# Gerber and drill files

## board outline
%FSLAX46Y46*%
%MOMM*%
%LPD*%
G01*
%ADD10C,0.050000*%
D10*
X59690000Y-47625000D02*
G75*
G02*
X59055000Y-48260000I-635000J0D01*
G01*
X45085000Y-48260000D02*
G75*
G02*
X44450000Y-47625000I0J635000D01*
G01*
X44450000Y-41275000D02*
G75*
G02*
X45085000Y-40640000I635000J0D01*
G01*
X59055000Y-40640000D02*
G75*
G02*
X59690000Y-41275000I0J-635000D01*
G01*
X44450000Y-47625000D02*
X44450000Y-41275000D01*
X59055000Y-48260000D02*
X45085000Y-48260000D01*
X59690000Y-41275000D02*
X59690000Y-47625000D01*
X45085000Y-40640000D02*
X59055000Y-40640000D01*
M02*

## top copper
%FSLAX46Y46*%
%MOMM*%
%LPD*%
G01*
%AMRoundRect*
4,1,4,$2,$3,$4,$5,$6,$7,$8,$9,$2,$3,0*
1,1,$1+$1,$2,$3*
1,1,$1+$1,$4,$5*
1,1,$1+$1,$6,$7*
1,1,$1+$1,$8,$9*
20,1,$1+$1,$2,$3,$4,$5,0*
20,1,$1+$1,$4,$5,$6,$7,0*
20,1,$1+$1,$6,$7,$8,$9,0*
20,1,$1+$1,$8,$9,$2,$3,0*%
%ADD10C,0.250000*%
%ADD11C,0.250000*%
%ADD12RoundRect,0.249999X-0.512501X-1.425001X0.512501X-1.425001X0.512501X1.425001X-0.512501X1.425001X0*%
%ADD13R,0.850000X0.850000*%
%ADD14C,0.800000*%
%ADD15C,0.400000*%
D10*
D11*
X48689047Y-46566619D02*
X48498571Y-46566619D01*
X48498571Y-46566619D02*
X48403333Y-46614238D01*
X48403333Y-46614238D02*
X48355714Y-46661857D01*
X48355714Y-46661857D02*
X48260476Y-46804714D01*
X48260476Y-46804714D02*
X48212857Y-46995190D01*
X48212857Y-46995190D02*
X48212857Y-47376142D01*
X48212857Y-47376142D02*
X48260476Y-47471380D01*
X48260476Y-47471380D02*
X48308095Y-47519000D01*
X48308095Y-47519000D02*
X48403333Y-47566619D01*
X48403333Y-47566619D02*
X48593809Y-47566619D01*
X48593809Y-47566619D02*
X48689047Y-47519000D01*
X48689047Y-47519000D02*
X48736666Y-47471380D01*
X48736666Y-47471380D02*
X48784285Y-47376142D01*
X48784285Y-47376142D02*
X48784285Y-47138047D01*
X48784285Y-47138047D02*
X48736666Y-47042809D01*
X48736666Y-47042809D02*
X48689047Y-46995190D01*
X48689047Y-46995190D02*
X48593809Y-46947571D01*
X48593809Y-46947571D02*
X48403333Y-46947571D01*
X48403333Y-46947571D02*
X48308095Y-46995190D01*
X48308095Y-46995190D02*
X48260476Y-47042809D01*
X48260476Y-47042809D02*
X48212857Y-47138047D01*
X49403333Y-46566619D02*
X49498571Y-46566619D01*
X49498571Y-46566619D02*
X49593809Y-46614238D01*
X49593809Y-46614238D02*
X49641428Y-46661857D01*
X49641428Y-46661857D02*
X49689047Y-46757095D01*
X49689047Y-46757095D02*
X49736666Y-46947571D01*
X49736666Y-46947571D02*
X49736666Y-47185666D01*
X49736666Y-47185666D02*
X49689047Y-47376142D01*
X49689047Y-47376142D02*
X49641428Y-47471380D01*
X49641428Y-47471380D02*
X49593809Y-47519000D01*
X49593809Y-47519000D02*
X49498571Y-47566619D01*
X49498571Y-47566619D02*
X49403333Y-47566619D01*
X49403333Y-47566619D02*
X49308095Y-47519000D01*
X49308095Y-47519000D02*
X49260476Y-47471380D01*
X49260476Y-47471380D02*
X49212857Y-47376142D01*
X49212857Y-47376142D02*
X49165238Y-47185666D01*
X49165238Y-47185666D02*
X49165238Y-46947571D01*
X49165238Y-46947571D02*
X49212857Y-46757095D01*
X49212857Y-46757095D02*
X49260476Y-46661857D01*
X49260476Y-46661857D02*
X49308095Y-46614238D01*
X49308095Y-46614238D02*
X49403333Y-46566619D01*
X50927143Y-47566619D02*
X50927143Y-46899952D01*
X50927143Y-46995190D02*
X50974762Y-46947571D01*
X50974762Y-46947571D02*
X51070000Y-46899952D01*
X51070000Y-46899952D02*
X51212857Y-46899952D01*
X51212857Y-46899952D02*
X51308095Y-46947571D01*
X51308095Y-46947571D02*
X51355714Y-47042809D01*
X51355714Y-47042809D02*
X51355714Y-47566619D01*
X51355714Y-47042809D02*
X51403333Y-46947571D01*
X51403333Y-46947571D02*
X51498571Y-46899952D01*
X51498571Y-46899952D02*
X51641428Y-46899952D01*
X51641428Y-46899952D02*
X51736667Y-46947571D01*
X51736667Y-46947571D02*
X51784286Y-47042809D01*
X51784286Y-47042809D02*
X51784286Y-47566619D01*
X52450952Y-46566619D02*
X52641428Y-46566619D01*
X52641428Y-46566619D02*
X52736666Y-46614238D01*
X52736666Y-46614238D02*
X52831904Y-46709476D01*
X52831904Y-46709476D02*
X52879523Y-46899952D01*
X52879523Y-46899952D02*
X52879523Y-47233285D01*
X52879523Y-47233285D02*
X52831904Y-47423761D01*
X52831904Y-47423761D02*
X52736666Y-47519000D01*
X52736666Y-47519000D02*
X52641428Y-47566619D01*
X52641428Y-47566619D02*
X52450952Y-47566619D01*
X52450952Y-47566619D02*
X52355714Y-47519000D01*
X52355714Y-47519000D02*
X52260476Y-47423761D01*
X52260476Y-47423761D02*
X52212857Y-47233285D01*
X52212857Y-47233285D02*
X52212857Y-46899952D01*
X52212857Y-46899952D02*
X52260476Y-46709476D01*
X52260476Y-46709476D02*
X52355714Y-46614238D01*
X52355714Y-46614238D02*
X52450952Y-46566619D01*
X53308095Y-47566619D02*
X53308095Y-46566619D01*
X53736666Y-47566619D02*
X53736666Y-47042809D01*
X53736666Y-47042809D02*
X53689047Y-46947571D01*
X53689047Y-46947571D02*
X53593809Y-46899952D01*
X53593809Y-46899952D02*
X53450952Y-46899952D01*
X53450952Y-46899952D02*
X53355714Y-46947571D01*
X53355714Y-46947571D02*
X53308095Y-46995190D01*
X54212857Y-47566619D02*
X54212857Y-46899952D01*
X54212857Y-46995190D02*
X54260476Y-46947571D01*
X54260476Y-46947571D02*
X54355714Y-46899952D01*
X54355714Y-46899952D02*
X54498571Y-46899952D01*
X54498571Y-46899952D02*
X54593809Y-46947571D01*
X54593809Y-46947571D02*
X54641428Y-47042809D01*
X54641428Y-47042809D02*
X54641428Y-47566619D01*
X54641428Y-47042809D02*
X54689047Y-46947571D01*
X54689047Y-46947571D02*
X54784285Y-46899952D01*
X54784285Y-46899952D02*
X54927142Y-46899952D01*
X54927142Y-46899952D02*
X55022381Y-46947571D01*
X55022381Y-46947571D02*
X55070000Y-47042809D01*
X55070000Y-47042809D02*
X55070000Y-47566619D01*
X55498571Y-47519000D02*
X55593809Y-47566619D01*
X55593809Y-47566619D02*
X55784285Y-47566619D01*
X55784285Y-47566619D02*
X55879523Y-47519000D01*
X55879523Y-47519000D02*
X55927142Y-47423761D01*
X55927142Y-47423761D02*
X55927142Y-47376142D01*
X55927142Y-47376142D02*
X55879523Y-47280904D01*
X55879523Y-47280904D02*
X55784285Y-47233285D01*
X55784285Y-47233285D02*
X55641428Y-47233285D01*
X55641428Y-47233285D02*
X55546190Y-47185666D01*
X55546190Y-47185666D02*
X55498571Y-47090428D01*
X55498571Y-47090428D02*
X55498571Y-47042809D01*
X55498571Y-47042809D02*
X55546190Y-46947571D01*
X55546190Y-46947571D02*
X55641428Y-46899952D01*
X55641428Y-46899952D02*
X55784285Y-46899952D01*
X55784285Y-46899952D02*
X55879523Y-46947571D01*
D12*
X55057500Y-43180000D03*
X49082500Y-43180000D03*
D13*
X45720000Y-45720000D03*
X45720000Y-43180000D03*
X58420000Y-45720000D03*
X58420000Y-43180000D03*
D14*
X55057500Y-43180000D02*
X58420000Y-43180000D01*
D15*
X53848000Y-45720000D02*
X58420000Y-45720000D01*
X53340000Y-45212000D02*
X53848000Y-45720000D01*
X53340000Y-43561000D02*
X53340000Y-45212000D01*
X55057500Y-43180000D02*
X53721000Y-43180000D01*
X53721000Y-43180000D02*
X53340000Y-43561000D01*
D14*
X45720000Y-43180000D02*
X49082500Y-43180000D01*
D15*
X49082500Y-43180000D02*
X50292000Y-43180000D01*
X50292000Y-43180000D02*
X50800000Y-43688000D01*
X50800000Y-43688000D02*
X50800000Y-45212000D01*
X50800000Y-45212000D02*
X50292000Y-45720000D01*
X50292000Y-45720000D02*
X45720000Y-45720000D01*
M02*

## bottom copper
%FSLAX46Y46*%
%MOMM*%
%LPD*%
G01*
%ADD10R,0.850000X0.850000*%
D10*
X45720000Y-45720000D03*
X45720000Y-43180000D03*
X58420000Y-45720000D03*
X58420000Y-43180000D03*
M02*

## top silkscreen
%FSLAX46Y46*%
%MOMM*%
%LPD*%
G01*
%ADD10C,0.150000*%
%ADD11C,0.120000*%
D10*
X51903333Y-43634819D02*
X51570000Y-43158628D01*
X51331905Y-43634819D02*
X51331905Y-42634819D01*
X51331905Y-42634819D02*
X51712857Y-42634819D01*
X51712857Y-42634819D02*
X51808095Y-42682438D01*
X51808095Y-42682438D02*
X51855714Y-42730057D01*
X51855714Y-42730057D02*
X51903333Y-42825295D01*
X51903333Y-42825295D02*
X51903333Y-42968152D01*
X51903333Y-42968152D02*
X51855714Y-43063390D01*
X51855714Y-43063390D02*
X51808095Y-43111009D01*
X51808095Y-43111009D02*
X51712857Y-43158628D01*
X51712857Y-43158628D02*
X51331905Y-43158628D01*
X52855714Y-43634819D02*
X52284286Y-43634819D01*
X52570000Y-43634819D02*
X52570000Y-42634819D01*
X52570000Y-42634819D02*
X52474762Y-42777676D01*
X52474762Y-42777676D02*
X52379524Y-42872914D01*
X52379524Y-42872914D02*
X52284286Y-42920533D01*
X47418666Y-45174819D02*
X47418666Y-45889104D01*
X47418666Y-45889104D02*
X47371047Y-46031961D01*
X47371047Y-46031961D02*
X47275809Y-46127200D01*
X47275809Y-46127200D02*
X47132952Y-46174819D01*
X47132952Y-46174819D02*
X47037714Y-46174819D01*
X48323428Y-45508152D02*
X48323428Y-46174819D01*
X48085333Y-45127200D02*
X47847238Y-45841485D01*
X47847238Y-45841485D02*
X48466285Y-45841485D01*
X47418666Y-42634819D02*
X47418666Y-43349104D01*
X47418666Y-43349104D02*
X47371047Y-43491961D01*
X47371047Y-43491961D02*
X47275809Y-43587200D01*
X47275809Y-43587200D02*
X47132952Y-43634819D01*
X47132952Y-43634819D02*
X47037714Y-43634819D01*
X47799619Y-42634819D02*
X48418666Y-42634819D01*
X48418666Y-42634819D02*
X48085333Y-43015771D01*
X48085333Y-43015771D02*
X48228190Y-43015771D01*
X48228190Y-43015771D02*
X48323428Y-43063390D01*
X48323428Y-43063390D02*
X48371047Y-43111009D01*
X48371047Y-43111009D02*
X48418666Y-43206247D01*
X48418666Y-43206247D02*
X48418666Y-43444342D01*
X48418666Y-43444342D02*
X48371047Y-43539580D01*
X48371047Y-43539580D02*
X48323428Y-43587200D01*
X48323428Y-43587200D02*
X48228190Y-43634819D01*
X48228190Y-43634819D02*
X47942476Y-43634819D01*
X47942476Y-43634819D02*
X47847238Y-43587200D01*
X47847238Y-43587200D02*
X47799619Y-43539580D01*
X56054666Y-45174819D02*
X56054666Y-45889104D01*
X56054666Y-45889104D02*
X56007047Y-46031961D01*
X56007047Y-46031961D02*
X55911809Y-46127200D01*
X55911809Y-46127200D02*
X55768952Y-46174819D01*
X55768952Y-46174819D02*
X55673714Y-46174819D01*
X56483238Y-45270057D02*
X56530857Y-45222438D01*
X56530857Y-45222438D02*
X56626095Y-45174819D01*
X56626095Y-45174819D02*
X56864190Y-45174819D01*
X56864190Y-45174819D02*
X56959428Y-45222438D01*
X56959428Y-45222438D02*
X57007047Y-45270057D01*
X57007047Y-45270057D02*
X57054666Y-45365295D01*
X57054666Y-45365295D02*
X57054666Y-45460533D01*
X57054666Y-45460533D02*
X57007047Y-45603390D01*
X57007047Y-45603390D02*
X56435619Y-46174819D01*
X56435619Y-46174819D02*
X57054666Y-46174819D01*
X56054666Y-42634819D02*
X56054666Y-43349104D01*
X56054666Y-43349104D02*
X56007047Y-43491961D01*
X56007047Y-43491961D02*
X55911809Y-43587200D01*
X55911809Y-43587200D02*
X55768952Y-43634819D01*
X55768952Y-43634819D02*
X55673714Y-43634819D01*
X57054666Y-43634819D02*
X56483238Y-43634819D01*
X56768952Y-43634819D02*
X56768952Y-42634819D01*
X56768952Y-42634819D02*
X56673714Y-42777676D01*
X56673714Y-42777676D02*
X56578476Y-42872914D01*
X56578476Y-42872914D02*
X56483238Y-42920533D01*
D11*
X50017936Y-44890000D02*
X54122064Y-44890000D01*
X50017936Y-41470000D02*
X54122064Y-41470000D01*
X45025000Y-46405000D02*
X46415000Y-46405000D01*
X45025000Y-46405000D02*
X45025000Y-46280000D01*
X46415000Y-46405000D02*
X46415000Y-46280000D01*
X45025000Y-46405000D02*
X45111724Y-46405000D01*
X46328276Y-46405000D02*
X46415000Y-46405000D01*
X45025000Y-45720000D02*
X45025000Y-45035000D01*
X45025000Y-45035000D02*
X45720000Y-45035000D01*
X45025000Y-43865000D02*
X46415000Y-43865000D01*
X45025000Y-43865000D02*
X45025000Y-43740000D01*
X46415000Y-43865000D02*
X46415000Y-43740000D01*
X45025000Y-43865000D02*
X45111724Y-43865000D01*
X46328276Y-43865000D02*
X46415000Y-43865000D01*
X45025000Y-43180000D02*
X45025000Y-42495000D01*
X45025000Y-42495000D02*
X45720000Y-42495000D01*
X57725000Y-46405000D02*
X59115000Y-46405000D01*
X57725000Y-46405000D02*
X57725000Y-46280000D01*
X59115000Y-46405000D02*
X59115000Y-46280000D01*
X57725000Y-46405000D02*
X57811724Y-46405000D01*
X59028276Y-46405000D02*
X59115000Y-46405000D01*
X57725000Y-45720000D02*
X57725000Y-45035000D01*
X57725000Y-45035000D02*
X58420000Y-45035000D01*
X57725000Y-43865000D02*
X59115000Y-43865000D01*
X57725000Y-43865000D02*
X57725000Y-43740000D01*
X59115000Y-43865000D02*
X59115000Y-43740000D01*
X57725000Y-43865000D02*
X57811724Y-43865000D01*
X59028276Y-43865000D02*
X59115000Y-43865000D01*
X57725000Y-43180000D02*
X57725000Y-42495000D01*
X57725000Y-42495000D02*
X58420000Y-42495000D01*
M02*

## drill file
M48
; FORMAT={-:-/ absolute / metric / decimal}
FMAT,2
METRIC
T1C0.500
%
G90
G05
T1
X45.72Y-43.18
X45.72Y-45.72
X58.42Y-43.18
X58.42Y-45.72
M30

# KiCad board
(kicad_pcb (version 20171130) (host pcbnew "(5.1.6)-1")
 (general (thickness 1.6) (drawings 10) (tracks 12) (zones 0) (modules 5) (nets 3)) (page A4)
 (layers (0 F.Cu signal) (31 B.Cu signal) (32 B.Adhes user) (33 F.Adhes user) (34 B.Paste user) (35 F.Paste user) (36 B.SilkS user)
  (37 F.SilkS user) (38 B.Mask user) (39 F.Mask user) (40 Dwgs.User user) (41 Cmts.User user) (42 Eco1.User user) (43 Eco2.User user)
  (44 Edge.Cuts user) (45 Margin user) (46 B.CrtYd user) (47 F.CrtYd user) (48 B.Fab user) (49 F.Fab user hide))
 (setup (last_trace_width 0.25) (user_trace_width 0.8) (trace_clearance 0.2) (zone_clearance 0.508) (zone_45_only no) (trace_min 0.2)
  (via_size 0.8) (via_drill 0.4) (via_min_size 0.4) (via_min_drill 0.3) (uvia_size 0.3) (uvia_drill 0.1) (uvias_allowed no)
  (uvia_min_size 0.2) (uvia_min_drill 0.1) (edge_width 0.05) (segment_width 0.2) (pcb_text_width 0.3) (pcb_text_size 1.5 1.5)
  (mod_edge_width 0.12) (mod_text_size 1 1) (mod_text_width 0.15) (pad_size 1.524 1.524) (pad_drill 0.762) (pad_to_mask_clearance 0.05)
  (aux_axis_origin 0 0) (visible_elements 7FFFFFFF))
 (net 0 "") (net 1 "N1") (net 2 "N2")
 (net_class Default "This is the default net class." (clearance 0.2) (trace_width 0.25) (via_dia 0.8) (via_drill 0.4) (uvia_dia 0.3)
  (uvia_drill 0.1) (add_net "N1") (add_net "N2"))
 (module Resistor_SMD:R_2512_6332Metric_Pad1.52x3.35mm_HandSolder (layer F.Cu) (at 52.07 43.18)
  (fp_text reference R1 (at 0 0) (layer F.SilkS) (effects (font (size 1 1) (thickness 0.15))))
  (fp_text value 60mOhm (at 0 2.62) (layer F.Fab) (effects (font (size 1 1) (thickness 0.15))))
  (fp_line (start -2.052064 1.71) (end 2.052064 1.71) (layer F.SilkS) (width 0.12))
  (fp_line (start -2.052064 -1.71) (end 2.052064 -1.71) (layer F.SilkS) (width 0.12))
  (pad 2 smd roundrect (at 2.9875 0) (size 1.525 3.35) (layers F.Cu F.Paste F.Mask) (roundrect_rratio 0.163934) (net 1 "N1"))
  (pad 1 smd roundrect (at -2.9875 0) (size 1.525 3.35) (layers F.Cu F.Paste F.Mask) (roundrect_rratio 0.163934) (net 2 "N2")))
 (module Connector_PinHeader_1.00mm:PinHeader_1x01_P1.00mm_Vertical (layer F.Cu) (at 45.72 45.72)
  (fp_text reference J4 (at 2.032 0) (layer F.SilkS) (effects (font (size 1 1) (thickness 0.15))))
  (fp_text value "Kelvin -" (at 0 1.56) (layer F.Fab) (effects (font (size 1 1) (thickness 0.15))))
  (fp_line (start -0.695 0.685) (end 0.695 0.685) (layer F.SilkS) (width 0.12))
  (fp_line (start -0.695 0.685) (end -0.695 0.56) (layer F.SilkS) (width 0.12))
  (fp_line (start 0.695 0.685) (end 0.695 0.56) (layer F.SilkS) (width 0.12))
  (fp_line (start -0.695 0.685) (end -0.608276 0.685) (layer F.SilkS) (width 0.12))
  (fp_line (start 0.608276 0.685) (end 0.695 0.685) (layer F.SilkS) (width 0.12))
  (fp_line (start -0.695 0) (end -0.695 -0.685) (layer F.SilkS) (width 0.12))
  (fp_line (start -0.695 -0.685) (end 0 -0.685) (layer F.SilkS) (width 0.12))
  (pad 1 thru_hole rect (at 0 0) (size 0.85 0.85) (drill 0.5) (layers *.Cu *.Mask) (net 2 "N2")))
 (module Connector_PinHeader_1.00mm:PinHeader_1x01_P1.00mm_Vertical (layer F.Cu) (at 45.72 43.18)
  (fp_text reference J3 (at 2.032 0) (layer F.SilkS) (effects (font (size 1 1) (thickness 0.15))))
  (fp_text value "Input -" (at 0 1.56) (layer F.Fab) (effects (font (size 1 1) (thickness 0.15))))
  (fp_line (start -0.695 0.685) (end 0.695 0.685) (layer F.SilkS) (width 0.12))
  (fp_line (start -0.695 0.685) (end -0.695 0.56) (layer F.SilkS) (width 0.12))
  (fp_line (start 0.695 0.685) (end 0.695 0.56) (layer F.SilkS) (width 0.12))
  (fp_line (start -0.695 0.685) (end -0.608276 0.685) (layer F.SilkS) (width 0.12))
  (fp_line (start 0.608276 0.685) (end 0.695 0.685) (layer F.SilkS) (width 0.12))
  (fp_line (start -0.695 0) (end -0.695 -0.685) (layer F.SilkS) (width 0.12))
  (fp_line (start -0.695 -0.685) (end 0 -0.685) (layer F.SilkS) (width 0.12))
  (pad 1 thru_hole rect (at 0 0) (size 0.85 0.85) (drill 0.5) (layers *.Cu *.Mask) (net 2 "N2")))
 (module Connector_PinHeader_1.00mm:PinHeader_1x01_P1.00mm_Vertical (layer F.Cu) (at 58.42 45.72)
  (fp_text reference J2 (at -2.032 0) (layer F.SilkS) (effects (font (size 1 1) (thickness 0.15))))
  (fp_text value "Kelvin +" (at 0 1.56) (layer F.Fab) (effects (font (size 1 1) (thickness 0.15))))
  (fp_line (start -0.695 0.685) (end 0.695 0.685) (layer F.SilkS) (width 0.12))
  (fp_line (start -0.695 0.685) (end -0.695 0.56) (layer F.SilkS) (width 0.12))
  (fp_line (start 0.695 0.685) (end 0.695 0.56) (layer F.SilkS) (width 0.12))
  (fp_line (start -0.695 0.685) (end -0.608276 0.685) (layer F.SilkS) (width 0.12))
  (fp_line (start 0.608276 0.685) (end 0.695 0.685) (layer F.SilkS) (width 0.12))
  (fp_line (start -0.695 0) (end -0.695 -0.685) (layer F.SilkS) (width 0.12))
  (fp_line (start -0.695 -0.685) (end 0 -0.685) (layer F.SilkS) (width 0.12))
  (pad 1 thru_hole rect (at 0 0) (size 0.85 0.85) (drill 0.5) (layers *.Cu *.Mask) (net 1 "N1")))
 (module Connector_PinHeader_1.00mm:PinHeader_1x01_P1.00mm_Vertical (layer F.Cu) (at 58.42 43.18)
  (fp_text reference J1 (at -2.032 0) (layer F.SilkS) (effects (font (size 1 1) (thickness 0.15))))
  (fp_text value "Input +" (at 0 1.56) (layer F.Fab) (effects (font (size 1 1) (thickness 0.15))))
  (fp_line (start -0.695 0.685) (end 0.695 0.685) (layer F.SilkS) (width 0.12))
  (fp_line (start -0.695 0.685) (end -0.695 0.56) (layer F.SilkS) (width 0.12))
  (fp_line (start 0.695 0.685) (end 0.695 0.56) (layer F.SilkS) (width 0.12))
  (fp_line (start -0.695 0.685) (end -0.608276 0.685) (layer F.SilkS) (width 0.12))
  (fp_line (start 0.608276 0.685) (end 0.695 0.685) (layer F.SilkS) (width 0.12))
  (fp_line (start -0.695 0) (end -0.695 -0.685) (layer F.SilkS) (width 0.12))
  (fp_line (start -0.695 -0.685) (end 0 -0.685) (layer F.SilkS) (width 0.12))
  (pad 1 thru_hole rect (at 0 0) (size 0.85 0.85) (drill 0.5) (layers *.Cu *.Mask) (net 1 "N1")))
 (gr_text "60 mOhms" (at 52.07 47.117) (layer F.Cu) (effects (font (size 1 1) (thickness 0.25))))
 (gr_arc (start 59.055 47.625) (end 59.055 48.26) (angle -90) (layer Edge.Cuts) (width 0.05))
 (gr_arc (start 45.085 47.625) (end 44.45 47.625) (angle -90) (layer Edge.Cuts) (width 0.05))
 (gr_arc (start 45.085 41.275) (end 45.085 40.64) (angle -90) (layer Edge.Cuts) (width 0.05))
 (gr_arc (start 59.055 41.275) (end 59.69 41.275) (angle -90) (layer Edge.Cuts) (width 0.05))
 (gr_line (start 44.45 47.625) (end 44.45 41.275) (layer Edge.Cuts) (width 0.05))
 (gr_line (start 59.055 48.26) (end 45.085 48.26) (layer Edge.Cuts) (width 0.05))
 (gr_line (start 59.69 41.275) (end 59.69 47.625) (layer Edge.Cuts) (width 0.05))
 (gr_line (start 45.085 40.64) (end 59.055 40.64) (layer Edge.Cuts) (width 0.05))
 (segment (start 55.0575 43.18) (end 58.42 43.18) (width 0.8) (layer F.Cu) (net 1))
 (segment (start 53.848 45.72) (end 58.42 45.72) (width 0.4) (layer F.Cu) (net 1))
 (segment (start 53.34 45.212) (end 53.848 45.72) (width 0.4) (layer F.Cu) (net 1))
 (segment (start 53.34 43.561) (end 53.34 45.212) (width 0.4) (layer F.Cu) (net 1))
 (segment (start 55.0575 43.18) (end 53.721 43.18) (width 0.4) (layer F.Cu) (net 1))
 (segment (start 53.721 43.18) (end 53.34 43.561) (width 0.4) (layer F.Cu) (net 1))
 (segment (start 45.72 43.18) (end 49.0825 43.18) (width 0.8) (layer F.Cu) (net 2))
 (segment (start 49.0825 43.18) (end 50.292 43.18) (width 0.4) (layer F.Cu) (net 2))
 (segment (start 50.292 43.18) (end 50.8 43.688) (width 0.4) (layer F.Cu) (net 2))
 (segment (start 50.8 43.688) (end 50.8 45.212) (width 0.4) (layer F.Cu) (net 2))
 (segment (start 50.8 45.212) (end 50.292 45.72) (width 0.4) (layer F.Cu) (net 2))
 (segment (start 50.292 45.72) (end 45.72 45.72) (width 0.4) (layer F.Cu) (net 2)))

